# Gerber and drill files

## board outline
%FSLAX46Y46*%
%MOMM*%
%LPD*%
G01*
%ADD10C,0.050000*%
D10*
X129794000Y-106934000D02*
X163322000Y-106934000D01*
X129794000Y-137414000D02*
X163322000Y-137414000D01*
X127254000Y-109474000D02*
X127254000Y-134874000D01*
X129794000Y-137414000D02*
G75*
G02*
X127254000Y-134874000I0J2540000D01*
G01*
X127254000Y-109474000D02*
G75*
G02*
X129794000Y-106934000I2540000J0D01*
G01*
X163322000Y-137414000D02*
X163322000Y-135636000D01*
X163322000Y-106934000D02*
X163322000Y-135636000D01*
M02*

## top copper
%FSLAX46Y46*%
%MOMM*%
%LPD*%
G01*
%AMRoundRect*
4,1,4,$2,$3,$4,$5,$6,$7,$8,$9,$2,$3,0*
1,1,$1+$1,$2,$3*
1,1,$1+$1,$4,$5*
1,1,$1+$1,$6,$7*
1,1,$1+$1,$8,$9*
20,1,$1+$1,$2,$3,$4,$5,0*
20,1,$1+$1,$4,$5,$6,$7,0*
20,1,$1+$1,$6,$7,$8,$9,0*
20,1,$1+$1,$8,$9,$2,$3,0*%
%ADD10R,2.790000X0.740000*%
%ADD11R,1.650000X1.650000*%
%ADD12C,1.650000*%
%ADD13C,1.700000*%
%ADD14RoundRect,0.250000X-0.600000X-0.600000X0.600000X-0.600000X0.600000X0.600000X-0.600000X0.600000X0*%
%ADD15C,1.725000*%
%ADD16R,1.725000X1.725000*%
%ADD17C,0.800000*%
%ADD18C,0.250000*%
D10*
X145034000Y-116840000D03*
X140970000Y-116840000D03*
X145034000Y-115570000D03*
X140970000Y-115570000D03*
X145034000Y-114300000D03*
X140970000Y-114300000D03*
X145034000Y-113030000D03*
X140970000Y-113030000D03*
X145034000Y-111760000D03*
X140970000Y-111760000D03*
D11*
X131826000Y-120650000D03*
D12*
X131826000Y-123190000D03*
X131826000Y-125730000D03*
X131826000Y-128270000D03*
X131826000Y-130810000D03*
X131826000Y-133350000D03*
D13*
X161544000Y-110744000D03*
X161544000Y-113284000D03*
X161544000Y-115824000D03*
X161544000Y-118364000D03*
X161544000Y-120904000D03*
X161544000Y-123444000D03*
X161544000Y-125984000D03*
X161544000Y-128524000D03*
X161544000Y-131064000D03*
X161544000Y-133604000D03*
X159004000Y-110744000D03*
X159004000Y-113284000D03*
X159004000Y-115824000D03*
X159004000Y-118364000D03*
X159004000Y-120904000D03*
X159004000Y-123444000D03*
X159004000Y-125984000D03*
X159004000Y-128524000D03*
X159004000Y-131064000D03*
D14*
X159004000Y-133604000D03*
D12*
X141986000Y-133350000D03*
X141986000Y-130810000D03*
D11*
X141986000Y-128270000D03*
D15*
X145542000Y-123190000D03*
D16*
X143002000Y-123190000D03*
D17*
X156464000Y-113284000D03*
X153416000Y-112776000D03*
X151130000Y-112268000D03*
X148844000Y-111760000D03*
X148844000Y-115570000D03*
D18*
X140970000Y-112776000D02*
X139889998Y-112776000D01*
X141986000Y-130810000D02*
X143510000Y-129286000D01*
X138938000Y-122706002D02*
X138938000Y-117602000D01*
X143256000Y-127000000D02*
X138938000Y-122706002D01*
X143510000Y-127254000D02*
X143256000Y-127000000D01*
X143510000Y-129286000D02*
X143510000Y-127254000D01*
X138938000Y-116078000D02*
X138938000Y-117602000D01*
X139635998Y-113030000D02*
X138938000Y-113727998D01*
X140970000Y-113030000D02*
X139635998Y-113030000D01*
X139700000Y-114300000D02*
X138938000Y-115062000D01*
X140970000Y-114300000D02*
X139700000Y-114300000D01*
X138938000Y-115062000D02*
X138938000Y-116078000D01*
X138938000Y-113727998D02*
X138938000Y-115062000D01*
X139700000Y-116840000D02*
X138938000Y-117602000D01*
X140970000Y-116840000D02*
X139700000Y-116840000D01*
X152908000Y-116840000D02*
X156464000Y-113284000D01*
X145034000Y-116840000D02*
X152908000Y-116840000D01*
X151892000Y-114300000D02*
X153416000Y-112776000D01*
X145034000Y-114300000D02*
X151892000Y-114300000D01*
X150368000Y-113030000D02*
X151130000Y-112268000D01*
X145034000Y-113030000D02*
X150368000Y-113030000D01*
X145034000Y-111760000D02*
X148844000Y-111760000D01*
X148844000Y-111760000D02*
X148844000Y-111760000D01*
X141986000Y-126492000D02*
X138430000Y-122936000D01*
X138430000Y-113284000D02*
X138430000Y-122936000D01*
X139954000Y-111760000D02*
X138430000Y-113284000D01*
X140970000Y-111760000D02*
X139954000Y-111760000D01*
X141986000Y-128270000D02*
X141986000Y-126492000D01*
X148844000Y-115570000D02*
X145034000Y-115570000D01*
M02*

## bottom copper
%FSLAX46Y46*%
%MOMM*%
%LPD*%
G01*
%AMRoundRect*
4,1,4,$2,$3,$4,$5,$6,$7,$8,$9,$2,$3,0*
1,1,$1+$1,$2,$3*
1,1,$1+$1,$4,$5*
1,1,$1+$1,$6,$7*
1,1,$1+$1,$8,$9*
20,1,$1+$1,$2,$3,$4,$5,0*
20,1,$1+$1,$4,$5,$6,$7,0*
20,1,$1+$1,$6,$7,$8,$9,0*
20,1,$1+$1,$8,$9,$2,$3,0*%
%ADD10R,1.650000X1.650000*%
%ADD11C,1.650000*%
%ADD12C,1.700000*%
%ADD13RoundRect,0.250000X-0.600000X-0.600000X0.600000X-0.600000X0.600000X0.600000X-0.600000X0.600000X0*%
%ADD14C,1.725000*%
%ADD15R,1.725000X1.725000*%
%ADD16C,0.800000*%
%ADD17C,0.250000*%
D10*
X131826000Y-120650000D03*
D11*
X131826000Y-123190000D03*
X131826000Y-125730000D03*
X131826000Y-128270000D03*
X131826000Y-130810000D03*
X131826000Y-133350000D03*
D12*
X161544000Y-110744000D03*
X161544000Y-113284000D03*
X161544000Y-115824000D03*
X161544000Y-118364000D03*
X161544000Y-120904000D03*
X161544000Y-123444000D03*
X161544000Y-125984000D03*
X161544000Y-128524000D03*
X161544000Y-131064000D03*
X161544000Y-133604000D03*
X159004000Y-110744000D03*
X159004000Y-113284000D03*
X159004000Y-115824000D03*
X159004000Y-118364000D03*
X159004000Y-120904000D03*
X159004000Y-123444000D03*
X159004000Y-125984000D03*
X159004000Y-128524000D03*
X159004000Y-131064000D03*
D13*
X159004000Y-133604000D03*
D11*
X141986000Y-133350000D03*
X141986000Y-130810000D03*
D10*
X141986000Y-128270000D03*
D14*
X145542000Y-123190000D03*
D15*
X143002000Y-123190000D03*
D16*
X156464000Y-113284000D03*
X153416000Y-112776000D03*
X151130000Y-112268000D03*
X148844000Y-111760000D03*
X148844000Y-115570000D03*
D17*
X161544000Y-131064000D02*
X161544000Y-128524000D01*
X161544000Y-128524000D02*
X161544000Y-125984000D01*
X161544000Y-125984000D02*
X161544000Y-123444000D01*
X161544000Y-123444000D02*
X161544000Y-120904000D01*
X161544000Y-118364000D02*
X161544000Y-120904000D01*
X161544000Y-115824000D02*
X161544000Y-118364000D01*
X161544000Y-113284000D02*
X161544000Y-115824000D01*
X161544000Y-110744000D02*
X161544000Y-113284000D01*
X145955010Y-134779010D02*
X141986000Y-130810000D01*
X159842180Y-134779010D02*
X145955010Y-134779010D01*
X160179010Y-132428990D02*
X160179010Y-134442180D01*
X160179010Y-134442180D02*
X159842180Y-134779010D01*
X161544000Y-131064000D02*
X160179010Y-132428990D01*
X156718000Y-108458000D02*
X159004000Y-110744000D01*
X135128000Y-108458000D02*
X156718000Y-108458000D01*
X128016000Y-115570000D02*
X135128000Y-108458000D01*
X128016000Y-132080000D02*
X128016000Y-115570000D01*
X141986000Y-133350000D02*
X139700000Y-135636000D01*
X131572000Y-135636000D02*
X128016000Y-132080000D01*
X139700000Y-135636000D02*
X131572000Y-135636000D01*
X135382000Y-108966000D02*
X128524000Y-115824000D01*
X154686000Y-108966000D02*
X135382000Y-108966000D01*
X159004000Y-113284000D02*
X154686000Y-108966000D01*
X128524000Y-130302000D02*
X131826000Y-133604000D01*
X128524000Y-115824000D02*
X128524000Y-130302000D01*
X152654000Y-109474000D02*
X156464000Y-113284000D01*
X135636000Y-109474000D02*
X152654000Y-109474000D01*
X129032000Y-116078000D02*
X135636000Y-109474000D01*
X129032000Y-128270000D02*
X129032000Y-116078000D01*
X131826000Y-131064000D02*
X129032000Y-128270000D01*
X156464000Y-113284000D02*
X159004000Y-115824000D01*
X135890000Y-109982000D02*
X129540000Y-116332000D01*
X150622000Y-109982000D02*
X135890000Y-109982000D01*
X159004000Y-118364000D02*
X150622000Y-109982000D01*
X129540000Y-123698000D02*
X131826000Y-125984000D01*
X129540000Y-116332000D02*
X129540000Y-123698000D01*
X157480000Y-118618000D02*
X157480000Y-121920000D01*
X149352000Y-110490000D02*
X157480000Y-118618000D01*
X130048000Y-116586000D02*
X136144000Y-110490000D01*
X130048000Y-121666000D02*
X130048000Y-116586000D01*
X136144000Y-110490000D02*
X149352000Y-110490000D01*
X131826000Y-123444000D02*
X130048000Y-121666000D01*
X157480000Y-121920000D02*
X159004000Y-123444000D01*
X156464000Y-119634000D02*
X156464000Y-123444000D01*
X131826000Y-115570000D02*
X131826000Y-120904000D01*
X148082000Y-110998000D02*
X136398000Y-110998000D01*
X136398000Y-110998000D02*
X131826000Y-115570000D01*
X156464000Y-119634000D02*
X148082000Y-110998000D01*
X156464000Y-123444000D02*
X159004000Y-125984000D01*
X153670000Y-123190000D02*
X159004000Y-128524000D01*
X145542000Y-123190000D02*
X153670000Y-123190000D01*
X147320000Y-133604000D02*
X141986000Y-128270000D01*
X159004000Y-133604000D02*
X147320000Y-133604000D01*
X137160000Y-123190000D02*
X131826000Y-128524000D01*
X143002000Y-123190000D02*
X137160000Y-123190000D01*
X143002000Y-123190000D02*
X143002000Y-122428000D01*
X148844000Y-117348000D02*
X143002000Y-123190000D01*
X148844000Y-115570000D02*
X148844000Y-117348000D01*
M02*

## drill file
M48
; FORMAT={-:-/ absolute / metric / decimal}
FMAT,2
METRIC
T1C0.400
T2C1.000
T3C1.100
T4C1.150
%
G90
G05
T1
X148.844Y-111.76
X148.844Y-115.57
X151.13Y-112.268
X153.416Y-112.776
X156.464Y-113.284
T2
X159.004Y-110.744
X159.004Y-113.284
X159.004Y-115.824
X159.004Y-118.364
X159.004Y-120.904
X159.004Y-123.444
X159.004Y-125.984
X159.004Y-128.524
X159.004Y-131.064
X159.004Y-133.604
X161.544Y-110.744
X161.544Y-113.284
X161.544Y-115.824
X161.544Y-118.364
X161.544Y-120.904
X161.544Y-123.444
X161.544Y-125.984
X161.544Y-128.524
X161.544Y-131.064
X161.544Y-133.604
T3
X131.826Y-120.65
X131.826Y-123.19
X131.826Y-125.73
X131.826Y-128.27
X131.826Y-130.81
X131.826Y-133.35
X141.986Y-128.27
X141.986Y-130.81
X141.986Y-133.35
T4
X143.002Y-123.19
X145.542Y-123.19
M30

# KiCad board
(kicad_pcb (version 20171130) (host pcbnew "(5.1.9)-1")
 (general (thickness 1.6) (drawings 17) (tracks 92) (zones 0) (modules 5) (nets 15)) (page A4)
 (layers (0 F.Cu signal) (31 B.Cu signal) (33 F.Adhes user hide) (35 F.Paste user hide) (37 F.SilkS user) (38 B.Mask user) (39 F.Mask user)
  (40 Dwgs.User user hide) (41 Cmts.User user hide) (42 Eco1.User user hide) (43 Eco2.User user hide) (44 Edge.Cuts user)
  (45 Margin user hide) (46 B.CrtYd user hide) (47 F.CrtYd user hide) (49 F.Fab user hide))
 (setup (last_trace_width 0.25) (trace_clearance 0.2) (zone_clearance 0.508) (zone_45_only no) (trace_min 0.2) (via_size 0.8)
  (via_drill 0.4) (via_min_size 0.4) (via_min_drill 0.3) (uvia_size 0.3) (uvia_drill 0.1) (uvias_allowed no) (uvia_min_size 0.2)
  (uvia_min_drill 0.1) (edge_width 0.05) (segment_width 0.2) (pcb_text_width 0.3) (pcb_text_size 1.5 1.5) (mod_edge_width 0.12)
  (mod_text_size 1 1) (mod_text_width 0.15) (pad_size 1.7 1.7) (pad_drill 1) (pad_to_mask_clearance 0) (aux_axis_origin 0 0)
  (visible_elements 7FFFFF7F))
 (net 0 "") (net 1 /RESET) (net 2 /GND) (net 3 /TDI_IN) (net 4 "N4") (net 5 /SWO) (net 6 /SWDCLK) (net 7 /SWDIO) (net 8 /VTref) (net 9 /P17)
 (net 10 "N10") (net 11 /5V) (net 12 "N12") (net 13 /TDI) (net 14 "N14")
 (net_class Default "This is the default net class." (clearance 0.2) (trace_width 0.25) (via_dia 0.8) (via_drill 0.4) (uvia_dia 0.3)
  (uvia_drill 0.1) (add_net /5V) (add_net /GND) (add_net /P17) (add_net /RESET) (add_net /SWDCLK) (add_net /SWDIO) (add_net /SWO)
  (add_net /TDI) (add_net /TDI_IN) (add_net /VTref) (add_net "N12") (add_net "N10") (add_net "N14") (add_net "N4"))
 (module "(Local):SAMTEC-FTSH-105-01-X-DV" (layer F.Cu) (at 143.002 114.3 270)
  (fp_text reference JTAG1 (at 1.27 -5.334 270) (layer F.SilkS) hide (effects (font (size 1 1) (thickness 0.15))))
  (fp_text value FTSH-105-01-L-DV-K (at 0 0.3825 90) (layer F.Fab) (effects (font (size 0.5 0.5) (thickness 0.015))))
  (pad 10 smd rect (at 2.54 -2.032 270) (size 0.74 2.79) (layers F.Cu F.Paste) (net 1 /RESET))
  (pad 9 smd rect (at 2.54 2.032 270) (size 0.74 2.79) (layers F.Cu F.Paste) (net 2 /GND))
  (pad 8 smd rect (at 1.27 -2.032 270) (size 0.74 2.79) (layers F.Cu F.Paste) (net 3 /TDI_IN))
  (pad 7 smd rect (at 1.27 2.032 270) (size 0.74 2.79) (layers F.Cu F.Paste) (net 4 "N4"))
  (pad 6 smd rect (at 0 -2.032 270) (size 0.74 2.79) (layers F.Cu F.Paste) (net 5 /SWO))
  (pad 5 smd rect (at 0 2.032 270) (size 0.74 2.79) (layers F.Cu F.Paste) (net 2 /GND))
  (pad 4 smd rect (at -1.27 -2.032 270) (size 0.74 2.79) (layers F.Cu F.Paste) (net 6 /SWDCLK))
  (pad 3 smd rect (at -1.27 2.032 270) (size 0.74 2.79) (layers F.Cu F.Paste) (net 2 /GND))
  (pad 2 smd rect (at -2.54 -2.032 270) (size 0.74 2.79) (layers F.Cu F.Paste) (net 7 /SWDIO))
  (pad 1 smd rect (at -2.54 2.032 270) (size 0.74 2.79) (layers F.Cu F.Paste) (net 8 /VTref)))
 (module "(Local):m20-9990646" (layer F.Cu) (at 131.826 120.65 270)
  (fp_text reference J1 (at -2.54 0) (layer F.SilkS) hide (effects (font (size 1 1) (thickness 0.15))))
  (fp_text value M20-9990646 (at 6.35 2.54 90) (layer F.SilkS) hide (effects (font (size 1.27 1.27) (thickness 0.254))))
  (pad 1 thru_hole rect (at 0 0 270) (size 1.65 1.65) (drill 1.1) (layers *.Cu *.Mask) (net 7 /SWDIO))
  (pad 2 thru_hole circle (at 2.54 0 270) (size 1.65 1.65) (drill 1.1) (layers *.Cu *.Mask) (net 6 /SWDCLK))
  (pad 3 thru_hole circle (at 5.08 0 270) (size 1.65 1.65) (drill 1.1) (layers *.Cu *.Mask) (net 5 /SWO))
  (pad 4 thru_hole circle (at 7.62 0 270) (size 1.65 1.65) (drill 1.1) (layers *.Cu *.Mask) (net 3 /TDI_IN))
  (pad 5 thru_hole circle (at 10.16 0 270) (size 1.65 1.65) (drill 1.1) (layers *.Cu *.Mask) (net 1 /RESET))
  (pad 6 thru_hole circle (at 12.7 0 270) (size 1.65 1.65) (drill 1.1) (layers *.Cu *.Mask) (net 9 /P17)))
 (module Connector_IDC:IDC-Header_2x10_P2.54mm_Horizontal (layer B.Cu) (at 159.004 133.604)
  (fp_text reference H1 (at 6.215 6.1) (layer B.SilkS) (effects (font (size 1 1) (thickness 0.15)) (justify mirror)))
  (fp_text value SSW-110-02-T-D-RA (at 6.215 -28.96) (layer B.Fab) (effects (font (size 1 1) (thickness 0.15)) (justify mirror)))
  (pad 20 thru_hole circle (at 2.54 -22.86) (size 1.7 1.7) (drill 1) (layers *.Cu *.Mask) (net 2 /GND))
  (pad 18 thru_hole circle (at 2.54 -20.32) (size 1.7 1.7) (drill 1) (layers *.Cu *.Mask) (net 2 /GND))
  (pad 16 thru_hole circle (at 2.54 -17.78) (size 1.7 1.7) (drill 1) (layers *.Cu *.Mask) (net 2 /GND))
  (pad 14 thru_hole circle (at 2.54 -15.24) (size 1.7 1.7) (drill 1) (layers *.Cu *.Mask) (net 2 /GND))
  (pad 12 thru_hole circle (at 2.54 -12.7) (size 1.7 1.7) (drill 1) (layers *.Cu *.Mask) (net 2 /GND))
  (pad 10 thru_hole circle (at 2.54 -10.16) (size 1.7 1.7) (drill 1) (layers *.Cu *.Mask) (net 2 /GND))
  (pad 8 thru_hole circle (at 2.54 -7.62) (size 1.7 1.7) (drill 1) (layers *.Cu *.Mask) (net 2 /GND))
  (pad 6 thru_hole circle (at 2.54 -5.08) (size 1.7 1.7) (drill 1) (layers *.Cu *.Mask) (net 2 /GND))
  (pad 4 thru_hole circle (at 2.54 -2.54) (size 1.7 1.7) (drill 1) (layers *.Cu *.Mask) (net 2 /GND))
  (pad 2 thru_hole circle (at 2.54 0) (size 1.7 1.7) (drill 1) (layers *.Cu *.Mask) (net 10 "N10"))
  (pad 19 thru_hole circle (at 0 -22.86) (size 1.7 1.7) (drill 1) (layers *.Cu *.Mask) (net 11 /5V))
  (pad 17 thru_hole circle (at 0 -20.32) (size 1.7 1.7) (drill 1) (layers *.Cu *.Mask) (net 9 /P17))
  (pad 15 thru_hole circle (at 0 -17.78) (size 1.7 1.7) (drill 1) (layers *.Cu *.Mask) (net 1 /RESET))
  (pad 13 thru_hole circle (at 0 -15.24) (size 1.7 1.7) (drill 1) (layers *.Cu *.Mask) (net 5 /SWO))
  (pad 11 thru_hole circle (at 0 -12.7) (size 1.7 1.7) (drill 1) (layers *.Cu *.Mask) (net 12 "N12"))
  (pad 9 thru_hole circle (at 0 -10.16) (size 1.7 1.7) (drill 1) (layers *.Cu *.Mask) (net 6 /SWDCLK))
  (pad 7 thru_hole circle (at 0 -7.62) (size 1.7 1.7) (drill 1) (layers *.Cu *.Mask) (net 7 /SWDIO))
  (pad 5 thru_hole circle (at 0 -5.08) (size 1.7 1.7) (drill 1) (layers *.Cu *.Mask) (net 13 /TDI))
  (pad 3 thru_hole circle (at 0 -2.54) (size 1.7 1.7) (drill 1) (layers *.Cu *.Mask) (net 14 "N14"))
  (pad 1 thru_hole roundrect (at 0 0) (size 1.7 1.7) (drill 1) (layers *.Cu *.Mask) (roundrect_rratio 0.1470588235294118) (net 8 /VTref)))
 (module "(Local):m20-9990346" (layer F.Cu) (at 141.986 128.27 270)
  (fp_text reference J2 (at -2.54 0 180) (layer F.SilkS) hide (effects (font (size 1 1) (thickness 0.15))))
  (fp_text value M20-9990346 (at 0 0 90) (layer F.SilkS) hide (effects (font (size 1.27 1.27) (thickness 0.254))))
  (pad 3 thru_hole circle (at 5.08 0 270) (size 1.65 1.65) (drill 1.1) (layers *.Cu *.Mask) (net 11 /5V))
  (pad 2 thru_hole circle (at 2.54 0 270) (size 1.65 1.65) (drill 1.1) (layers *.Cu *.Mask) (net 2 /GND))
  (pad 1 thru_hole rect (at 0 0 270) (size 1.65 1.65) (drill 1.1) (layers *.Cu *.Mask) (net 8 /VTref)))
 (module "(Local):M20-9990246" (layer F.Cu) (at 143.002 123.19)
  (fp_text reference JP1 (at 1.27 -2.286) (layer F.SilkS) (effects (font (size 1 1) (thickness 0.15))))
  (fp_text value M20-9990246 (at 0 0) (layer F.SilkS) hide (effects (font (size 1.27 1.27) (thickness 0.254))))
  (pad 2 thru_hole circle (at 2.54 0) (size 1.725 1.725) (drill 1.15) (layers *.Cu *.Mask) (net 13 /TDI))
  (pad 1 thru_hole rect (at 0 0) (size 1.725 1.725) (drill 1.15) (layers *.Cu *.Mask) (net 3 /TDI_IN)))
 (gr_line (start 129.794 106.934) (end 163.322 106.934) (layer Edge.Cuts) (width 0.05))
 (gr_line (start 129.794 137.414) (end 163.322 137.414) (layer Edge.Cuts) (width 0.05))
 (gr_line (start 127.254 109.474) (end 127.254 134.874) (layer Edge.Cuts) (width 0.05))
 (gr_arc (start 129.794 134.874) (end 127.254 134.874) (angle -90) (layer Edge.Cuts) (width 0.05))
 (gr_arc (start 129.794 109.474) (end 129.794 106.934) (angle -90) (layer Edge.Cuts) (width 0.05))
 (gr_line (start 163.322 137.414) (end 163.322 135.636) (layer Edge.Cuts) (width 0.05))
 (gr_line (start 163.322 106.934) (end 163.322 135.636) (layer Edge.Cuts) (width 0.05))
 (segment (start 161.544 131.064) (end 161.544 128.524) (width 0.25) (layer B.Cu) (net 2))
 (segment (start 161.544 128.524) (end 161.544 125.984) (width 0.25) (layer B.Cu) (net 2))
 (segment (start 161.544 125.984) (end 161.544 123.444) (width 0.25) (layer B.Cu) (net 2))
 (segment (start 161.544 123.444) (end 161.544 120.904) (width 0.25) (layer B.Cu) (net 2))
 (segment (start 161.544 118.364) (end 161.544 120.904) (width 0.25) (layer B.Cu) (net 2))
 (segment (start 161.544 115.824) (end 161.544 118.364) (width 0.25) (layer B.Cu) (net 2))
 (segment (start 161.544 113.284) (end 161.544 115.824) (width 0.25) (layer B.Cu) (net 2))
 (segment (start 161.544 110.744) (end 161.544 113.284) (width 0.25) (layer B.Cu) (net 2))
 (segment (start 145.95501 134.77901) (end 141.986 130.81) (width 0.25) (layer B.Cu) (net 2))
 (segment (start 159.84218 134.77901) (end 145.95501 134.77901) (width 0.25) (layer B.Cu) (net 2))
 (segment (start 160.17901 132.42899) (end 160.17901 134.44218) (width 0.25) (layer B.Cu) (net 2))
 (segment (start 160.17901 134.44218) (end 159.84218 134.77901) (width 0.25) (layer B.Cu) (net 2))
 (segment (start 161.544 131.064) (end 160.17901 132.42899) (width 0.25) (layer B.Cu) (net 2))
 (segment (start 140.97 112.776) (end 139.889998 112.776) (width 0.25) (layer F.Cu) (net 2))
 (segment (start 141.986 130.81) (end 143.51 129.286) (width 0.25) (layer F.Cu) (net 2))
 (segment (start 138.938 122.706002) (end 138.938 117.602) (width 0.25) (layer F.Cu) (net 2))
 (segment (start 143.256 127) (end 138.938 122.706002) (width 0.25) (layer F.Cu) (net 2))
 (segment (start 143.51 127.254) (end 143.256 127) (width 0.25) (layer F.Cu) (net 2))
 (segment (start 143.51 129.286) (end 143.51 127.254) (width 0.25) (layer F.Cu) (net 2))
 (segment (start 138.938 116.078) (end 138.938 117.602) (width 0.25) (layer F.Cu) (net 2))
 (segment (start 139.635998 113.03) (end 138.938 113.727998) (width 0.25) (layer F.Cu) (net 2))
 (segment (start 140.97 113.03) (end 139.635998 113.03) (width 0.25) (layer F.Cu) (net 2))
 (segment (start 139.7 114.3) (end 138.938 115.062) (width 0.25) (layer F.Cu) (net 2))
 (segment (start 140.97 114.3) (end 139.7 114.3) (width 0.25) (layer F.Cu) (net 2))
 (segment (start 138.938 115.062) (end 138.938 116.078) (width 0.25) (layer F.Cu) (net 2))
 (segment (start 138.938 113.727998) (end 138.938 115.062) (width 0.25) (layer F.Cu) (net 2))
 (segment (start 139.7 116.84) (end 138.938 117.602) (width 0.25) (layer F.Cu) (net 2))
 (segment (start 140.97 116.84) (end 139.7 116.84) (width 0.25) (layer F.Cu) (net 2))
 (segment (start 156.718 108.458) (end 159.004 110.744) (width 0.25) (layer B.Cu) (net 11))
 (segment (start 135.128 108.458) (end 156.718 108.458) (width 0.25) (layer B.Cu) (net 11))
 (segment (start 128.016 115.57) (end 135.128 108.458) (width 0.25) (layer B.Cu) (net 11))
 (segment (start 128.016 132.08) (end 128.016 115.57) (width 0.25) (layer B.Cu) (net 11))
 (segment (start 141.986 133.35) (end 139.7 135.636) (width 0.25) (layer B.Cu) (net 11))
 (segment (start 131.572 135.636) (end 128.016 132.08) (width 0.25) (layer B.Cu) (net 11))
 (segment (start 139.7 135.636) (end 131.572 135.636) (width 0.25) (layer B.Cu) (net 11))
 (segment (start 135.382 108.966) (end 128.524 115.824) (width 0.25) (layer B.Cu) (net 9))
 (segment (start 154.686 108.966) (end 135.382 108.966) (width 0.25) (layer B.Cu) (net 9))
 (segment (start 159.004 113.284) (end 154.686 108.966) (width 0.25) (layer B.Cu) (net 9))
 (segment (start 128.524 130.302) (end 131.826 133.604) (width 0.25) (layer B.Cu) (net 9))
 (segment (start 128.524 115.824) (end 128.524 130.302) (width 0.25) (layer B.Cu) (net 9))
 (segment (start 152.654 109.474) (end 156.464 113.284) (width 0.25) (layer B.Cu) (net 1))
 (segment (start 135.636 109.474) (end 152.654 109.474) (width 0.25) (layer B.Cu) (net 1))
 (segment (start 129.032 116.078) (end 135.636 109.474) (width 0.25) (layer B.Cu) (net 1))
 (segment (start 129.032 128.27) (end 129.032 116.078) (width 0.25) (layer B.Cu) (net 1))
 (segment (start 131.826 131.064) (end 129.032 128.27) (width 0.25) (layer B.Cu) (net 1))
 (segment (start 156.464 113.284) (end 159.004 115.824) (width 0.25) (layer B.Cu) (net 1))
 (via (at 156.464 113.284) (size 0.8) (drill 0.4) (layers F.Cu B.Cu) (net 1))
 (segment (start 152.908 116.84) (end 156.464 113.284) (width 0.25) (layer F.Cu) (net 1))
 (segment (start 145.034 116.84) (end 152.908 116.84) (width 0.25) (layer F.Cu) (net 1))
 (via (at 153.416 112.776) (size 0.8) (drill 0.4) (layers F.Cu B.Cu) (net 5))
 (segment (start 135.89 109.982) (end 129.54 116.332) (width 0.25) (layer B.Cu) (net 5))
 (segment (start 150.622 109.982) (end 135.89 109.982) (width 0.25) (layer B.Cu) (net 5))
 (segment (start 159.004 118.364) (end 150.622 109.982) (width 0.25) (layer B.Cu) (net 5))
 (segment (start 129.54 123.698) (end 131.826 125.984) (width 0.25) (layer B.Cu) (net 5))
 (segment (start 129.54 116.332) (end 129.54 123.698) (width 0.25) (layer B.Cu) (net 5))
 (segment (start 151.892 114.3) (end 153.416 112.776) (width 0.25) (layer F.Cu) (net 5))
 (segment (start 145.034 114.3) (end 151.892 114.3) (width 0.25) (layer F.Cu) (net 5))
 (via (at 151.13 112.268) (size 0.8) (drill 0.4) (layers F.Cu B.Cu) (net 6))
 (segment (start 157.48 118.618) (end 157.48 121.92) (width 0.25) (layer B.Cu) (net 6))
 (segment (start 149.352 110.49) (end 157.48 118.618) (width 0.25) (layer B.Cu) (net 6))
 (segment (start 130.048 116.586) (end 136.144 110.49) (width 0.25) (layer B.Cu) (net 6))
 (segment (start 130.048 121.666) (end 130.048 116.586) (width 0.25) (layer B.Cu) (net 6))
 (segment (start 136.144 110.49) (end 149.352 110.49) (width 0.25) (layer B.Cu) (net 6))
 (segment (start 131.826 123.444) (end 130.048 121.666) (width 0.25) (layer B.Cu) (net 6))
 (segment (start 157.48 121.92) (end 159.004 123.444) (width 0.25) (layer B.Cu) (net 6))
 (segment (start 150.368 113.03) (end 151.13 112.268) (width 0.25) (layer F.Cu) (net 6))
 (segment (start 145.034 113.03) (end 150.368 113.03) (width 0.25) (layer F.Cu) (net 6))
 (segment (start 145.034 111.76) (end 148.844 111.76) (width 0.25) (layer F.Cu) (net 7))
 (segment (start 148.844 111.76) (end 148.844 111.76) (width 0.25) (layer F.Cu) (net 7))
 (via (at 148.844 111.76) (size 0.8) (drill 0.4) (layers F.Cu B.Cu) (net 7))
 (segment (start 156.464 119.634) (end 156.464 123.444) (width 0.25) (layer B.Cu) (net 7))
 (segment (start 131.826 115.57) (end 131.826 120.904) (width 0.25) (layer B.Cu) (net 7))
 (segment (start 148.082 110.998) (end 136.398 110.998) (width 0.25) (layer B.Cu) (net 7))
 (segment (start 136.398 110.998) (end 131.826 115.57) (width 0.25) (layer B.Cu) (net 7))
 (segment (start 156.464 119.634) (end 148.082 110.998) (width 0.25) (layer B.Cu) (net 7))
 (segment (start 156.464 123.444) (end 159.004 125.984) (width 0.25) (layer B.Cu) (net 7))
 (segment (start 153.67 123.19) (end 159.004 128.524) (width 0.25) (layer B.Cu) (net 13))
 (segment (start 145.542 123.19) (end 153.67 123.19) (width 0.25) (layer B.Cu) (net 13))
 (segment (start 147.32 133.604) (end 141.986 128.27) (width 0.25) (layer B.Cu) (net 8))
 (segment (start 159.004 133.604) (end 147.32 133.604) (width 0.25) (layer B.Cu) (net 8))
 (segment (start 141.986 126.492) (end 138.43 122.936) (width 0.25) (layer F.Cu) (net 8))
 (segment (start 138.43 113.284) (end 138.43 122.936) (width 0.25) (layer F.Cu) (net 8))
 (segment (start 139.954 111.76) (end 138.43 113.284) (width 0.25) (layer F.Cu) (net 8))
 (segment (start 140.97 111.76) (end 139.954 111.76) (width 0.25) (layer F.Cu) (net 8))
 (segment (start 141.986 128.27) (end 141.986 126.492) (width 0.25) (layer F.Cu) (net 8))
 (segment (start 137.16 123.19) (end 131.826 128.524) (width 0.25) (layer B.Cu) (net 3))
 (segment (start 143.002 123.19) (end 137.16 123.19) (width 0.25) (layer B.Cu) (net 3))
 (segment (start 143.002 123.19) (end 143.002 122.428) (width 0.25) (layer B.Cu) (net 3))
 (via (at 148.844 115.57) (size 0.8) (drill 0.4) (layers F.Cu B.Cu) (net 3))
 (segment (start 148.844 115.57) (end 145.034 115.57) (width 0.25) (layer F.Cu) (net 3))
 (segment (start 148.844 117.348) (end 143.002 123.19) (width 0.25) (layer B.Cu) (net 3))
 (segment (start 148.844 115.57) (end 148.844 117.348) (width 0.25) (layer B.Cu) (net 3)))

